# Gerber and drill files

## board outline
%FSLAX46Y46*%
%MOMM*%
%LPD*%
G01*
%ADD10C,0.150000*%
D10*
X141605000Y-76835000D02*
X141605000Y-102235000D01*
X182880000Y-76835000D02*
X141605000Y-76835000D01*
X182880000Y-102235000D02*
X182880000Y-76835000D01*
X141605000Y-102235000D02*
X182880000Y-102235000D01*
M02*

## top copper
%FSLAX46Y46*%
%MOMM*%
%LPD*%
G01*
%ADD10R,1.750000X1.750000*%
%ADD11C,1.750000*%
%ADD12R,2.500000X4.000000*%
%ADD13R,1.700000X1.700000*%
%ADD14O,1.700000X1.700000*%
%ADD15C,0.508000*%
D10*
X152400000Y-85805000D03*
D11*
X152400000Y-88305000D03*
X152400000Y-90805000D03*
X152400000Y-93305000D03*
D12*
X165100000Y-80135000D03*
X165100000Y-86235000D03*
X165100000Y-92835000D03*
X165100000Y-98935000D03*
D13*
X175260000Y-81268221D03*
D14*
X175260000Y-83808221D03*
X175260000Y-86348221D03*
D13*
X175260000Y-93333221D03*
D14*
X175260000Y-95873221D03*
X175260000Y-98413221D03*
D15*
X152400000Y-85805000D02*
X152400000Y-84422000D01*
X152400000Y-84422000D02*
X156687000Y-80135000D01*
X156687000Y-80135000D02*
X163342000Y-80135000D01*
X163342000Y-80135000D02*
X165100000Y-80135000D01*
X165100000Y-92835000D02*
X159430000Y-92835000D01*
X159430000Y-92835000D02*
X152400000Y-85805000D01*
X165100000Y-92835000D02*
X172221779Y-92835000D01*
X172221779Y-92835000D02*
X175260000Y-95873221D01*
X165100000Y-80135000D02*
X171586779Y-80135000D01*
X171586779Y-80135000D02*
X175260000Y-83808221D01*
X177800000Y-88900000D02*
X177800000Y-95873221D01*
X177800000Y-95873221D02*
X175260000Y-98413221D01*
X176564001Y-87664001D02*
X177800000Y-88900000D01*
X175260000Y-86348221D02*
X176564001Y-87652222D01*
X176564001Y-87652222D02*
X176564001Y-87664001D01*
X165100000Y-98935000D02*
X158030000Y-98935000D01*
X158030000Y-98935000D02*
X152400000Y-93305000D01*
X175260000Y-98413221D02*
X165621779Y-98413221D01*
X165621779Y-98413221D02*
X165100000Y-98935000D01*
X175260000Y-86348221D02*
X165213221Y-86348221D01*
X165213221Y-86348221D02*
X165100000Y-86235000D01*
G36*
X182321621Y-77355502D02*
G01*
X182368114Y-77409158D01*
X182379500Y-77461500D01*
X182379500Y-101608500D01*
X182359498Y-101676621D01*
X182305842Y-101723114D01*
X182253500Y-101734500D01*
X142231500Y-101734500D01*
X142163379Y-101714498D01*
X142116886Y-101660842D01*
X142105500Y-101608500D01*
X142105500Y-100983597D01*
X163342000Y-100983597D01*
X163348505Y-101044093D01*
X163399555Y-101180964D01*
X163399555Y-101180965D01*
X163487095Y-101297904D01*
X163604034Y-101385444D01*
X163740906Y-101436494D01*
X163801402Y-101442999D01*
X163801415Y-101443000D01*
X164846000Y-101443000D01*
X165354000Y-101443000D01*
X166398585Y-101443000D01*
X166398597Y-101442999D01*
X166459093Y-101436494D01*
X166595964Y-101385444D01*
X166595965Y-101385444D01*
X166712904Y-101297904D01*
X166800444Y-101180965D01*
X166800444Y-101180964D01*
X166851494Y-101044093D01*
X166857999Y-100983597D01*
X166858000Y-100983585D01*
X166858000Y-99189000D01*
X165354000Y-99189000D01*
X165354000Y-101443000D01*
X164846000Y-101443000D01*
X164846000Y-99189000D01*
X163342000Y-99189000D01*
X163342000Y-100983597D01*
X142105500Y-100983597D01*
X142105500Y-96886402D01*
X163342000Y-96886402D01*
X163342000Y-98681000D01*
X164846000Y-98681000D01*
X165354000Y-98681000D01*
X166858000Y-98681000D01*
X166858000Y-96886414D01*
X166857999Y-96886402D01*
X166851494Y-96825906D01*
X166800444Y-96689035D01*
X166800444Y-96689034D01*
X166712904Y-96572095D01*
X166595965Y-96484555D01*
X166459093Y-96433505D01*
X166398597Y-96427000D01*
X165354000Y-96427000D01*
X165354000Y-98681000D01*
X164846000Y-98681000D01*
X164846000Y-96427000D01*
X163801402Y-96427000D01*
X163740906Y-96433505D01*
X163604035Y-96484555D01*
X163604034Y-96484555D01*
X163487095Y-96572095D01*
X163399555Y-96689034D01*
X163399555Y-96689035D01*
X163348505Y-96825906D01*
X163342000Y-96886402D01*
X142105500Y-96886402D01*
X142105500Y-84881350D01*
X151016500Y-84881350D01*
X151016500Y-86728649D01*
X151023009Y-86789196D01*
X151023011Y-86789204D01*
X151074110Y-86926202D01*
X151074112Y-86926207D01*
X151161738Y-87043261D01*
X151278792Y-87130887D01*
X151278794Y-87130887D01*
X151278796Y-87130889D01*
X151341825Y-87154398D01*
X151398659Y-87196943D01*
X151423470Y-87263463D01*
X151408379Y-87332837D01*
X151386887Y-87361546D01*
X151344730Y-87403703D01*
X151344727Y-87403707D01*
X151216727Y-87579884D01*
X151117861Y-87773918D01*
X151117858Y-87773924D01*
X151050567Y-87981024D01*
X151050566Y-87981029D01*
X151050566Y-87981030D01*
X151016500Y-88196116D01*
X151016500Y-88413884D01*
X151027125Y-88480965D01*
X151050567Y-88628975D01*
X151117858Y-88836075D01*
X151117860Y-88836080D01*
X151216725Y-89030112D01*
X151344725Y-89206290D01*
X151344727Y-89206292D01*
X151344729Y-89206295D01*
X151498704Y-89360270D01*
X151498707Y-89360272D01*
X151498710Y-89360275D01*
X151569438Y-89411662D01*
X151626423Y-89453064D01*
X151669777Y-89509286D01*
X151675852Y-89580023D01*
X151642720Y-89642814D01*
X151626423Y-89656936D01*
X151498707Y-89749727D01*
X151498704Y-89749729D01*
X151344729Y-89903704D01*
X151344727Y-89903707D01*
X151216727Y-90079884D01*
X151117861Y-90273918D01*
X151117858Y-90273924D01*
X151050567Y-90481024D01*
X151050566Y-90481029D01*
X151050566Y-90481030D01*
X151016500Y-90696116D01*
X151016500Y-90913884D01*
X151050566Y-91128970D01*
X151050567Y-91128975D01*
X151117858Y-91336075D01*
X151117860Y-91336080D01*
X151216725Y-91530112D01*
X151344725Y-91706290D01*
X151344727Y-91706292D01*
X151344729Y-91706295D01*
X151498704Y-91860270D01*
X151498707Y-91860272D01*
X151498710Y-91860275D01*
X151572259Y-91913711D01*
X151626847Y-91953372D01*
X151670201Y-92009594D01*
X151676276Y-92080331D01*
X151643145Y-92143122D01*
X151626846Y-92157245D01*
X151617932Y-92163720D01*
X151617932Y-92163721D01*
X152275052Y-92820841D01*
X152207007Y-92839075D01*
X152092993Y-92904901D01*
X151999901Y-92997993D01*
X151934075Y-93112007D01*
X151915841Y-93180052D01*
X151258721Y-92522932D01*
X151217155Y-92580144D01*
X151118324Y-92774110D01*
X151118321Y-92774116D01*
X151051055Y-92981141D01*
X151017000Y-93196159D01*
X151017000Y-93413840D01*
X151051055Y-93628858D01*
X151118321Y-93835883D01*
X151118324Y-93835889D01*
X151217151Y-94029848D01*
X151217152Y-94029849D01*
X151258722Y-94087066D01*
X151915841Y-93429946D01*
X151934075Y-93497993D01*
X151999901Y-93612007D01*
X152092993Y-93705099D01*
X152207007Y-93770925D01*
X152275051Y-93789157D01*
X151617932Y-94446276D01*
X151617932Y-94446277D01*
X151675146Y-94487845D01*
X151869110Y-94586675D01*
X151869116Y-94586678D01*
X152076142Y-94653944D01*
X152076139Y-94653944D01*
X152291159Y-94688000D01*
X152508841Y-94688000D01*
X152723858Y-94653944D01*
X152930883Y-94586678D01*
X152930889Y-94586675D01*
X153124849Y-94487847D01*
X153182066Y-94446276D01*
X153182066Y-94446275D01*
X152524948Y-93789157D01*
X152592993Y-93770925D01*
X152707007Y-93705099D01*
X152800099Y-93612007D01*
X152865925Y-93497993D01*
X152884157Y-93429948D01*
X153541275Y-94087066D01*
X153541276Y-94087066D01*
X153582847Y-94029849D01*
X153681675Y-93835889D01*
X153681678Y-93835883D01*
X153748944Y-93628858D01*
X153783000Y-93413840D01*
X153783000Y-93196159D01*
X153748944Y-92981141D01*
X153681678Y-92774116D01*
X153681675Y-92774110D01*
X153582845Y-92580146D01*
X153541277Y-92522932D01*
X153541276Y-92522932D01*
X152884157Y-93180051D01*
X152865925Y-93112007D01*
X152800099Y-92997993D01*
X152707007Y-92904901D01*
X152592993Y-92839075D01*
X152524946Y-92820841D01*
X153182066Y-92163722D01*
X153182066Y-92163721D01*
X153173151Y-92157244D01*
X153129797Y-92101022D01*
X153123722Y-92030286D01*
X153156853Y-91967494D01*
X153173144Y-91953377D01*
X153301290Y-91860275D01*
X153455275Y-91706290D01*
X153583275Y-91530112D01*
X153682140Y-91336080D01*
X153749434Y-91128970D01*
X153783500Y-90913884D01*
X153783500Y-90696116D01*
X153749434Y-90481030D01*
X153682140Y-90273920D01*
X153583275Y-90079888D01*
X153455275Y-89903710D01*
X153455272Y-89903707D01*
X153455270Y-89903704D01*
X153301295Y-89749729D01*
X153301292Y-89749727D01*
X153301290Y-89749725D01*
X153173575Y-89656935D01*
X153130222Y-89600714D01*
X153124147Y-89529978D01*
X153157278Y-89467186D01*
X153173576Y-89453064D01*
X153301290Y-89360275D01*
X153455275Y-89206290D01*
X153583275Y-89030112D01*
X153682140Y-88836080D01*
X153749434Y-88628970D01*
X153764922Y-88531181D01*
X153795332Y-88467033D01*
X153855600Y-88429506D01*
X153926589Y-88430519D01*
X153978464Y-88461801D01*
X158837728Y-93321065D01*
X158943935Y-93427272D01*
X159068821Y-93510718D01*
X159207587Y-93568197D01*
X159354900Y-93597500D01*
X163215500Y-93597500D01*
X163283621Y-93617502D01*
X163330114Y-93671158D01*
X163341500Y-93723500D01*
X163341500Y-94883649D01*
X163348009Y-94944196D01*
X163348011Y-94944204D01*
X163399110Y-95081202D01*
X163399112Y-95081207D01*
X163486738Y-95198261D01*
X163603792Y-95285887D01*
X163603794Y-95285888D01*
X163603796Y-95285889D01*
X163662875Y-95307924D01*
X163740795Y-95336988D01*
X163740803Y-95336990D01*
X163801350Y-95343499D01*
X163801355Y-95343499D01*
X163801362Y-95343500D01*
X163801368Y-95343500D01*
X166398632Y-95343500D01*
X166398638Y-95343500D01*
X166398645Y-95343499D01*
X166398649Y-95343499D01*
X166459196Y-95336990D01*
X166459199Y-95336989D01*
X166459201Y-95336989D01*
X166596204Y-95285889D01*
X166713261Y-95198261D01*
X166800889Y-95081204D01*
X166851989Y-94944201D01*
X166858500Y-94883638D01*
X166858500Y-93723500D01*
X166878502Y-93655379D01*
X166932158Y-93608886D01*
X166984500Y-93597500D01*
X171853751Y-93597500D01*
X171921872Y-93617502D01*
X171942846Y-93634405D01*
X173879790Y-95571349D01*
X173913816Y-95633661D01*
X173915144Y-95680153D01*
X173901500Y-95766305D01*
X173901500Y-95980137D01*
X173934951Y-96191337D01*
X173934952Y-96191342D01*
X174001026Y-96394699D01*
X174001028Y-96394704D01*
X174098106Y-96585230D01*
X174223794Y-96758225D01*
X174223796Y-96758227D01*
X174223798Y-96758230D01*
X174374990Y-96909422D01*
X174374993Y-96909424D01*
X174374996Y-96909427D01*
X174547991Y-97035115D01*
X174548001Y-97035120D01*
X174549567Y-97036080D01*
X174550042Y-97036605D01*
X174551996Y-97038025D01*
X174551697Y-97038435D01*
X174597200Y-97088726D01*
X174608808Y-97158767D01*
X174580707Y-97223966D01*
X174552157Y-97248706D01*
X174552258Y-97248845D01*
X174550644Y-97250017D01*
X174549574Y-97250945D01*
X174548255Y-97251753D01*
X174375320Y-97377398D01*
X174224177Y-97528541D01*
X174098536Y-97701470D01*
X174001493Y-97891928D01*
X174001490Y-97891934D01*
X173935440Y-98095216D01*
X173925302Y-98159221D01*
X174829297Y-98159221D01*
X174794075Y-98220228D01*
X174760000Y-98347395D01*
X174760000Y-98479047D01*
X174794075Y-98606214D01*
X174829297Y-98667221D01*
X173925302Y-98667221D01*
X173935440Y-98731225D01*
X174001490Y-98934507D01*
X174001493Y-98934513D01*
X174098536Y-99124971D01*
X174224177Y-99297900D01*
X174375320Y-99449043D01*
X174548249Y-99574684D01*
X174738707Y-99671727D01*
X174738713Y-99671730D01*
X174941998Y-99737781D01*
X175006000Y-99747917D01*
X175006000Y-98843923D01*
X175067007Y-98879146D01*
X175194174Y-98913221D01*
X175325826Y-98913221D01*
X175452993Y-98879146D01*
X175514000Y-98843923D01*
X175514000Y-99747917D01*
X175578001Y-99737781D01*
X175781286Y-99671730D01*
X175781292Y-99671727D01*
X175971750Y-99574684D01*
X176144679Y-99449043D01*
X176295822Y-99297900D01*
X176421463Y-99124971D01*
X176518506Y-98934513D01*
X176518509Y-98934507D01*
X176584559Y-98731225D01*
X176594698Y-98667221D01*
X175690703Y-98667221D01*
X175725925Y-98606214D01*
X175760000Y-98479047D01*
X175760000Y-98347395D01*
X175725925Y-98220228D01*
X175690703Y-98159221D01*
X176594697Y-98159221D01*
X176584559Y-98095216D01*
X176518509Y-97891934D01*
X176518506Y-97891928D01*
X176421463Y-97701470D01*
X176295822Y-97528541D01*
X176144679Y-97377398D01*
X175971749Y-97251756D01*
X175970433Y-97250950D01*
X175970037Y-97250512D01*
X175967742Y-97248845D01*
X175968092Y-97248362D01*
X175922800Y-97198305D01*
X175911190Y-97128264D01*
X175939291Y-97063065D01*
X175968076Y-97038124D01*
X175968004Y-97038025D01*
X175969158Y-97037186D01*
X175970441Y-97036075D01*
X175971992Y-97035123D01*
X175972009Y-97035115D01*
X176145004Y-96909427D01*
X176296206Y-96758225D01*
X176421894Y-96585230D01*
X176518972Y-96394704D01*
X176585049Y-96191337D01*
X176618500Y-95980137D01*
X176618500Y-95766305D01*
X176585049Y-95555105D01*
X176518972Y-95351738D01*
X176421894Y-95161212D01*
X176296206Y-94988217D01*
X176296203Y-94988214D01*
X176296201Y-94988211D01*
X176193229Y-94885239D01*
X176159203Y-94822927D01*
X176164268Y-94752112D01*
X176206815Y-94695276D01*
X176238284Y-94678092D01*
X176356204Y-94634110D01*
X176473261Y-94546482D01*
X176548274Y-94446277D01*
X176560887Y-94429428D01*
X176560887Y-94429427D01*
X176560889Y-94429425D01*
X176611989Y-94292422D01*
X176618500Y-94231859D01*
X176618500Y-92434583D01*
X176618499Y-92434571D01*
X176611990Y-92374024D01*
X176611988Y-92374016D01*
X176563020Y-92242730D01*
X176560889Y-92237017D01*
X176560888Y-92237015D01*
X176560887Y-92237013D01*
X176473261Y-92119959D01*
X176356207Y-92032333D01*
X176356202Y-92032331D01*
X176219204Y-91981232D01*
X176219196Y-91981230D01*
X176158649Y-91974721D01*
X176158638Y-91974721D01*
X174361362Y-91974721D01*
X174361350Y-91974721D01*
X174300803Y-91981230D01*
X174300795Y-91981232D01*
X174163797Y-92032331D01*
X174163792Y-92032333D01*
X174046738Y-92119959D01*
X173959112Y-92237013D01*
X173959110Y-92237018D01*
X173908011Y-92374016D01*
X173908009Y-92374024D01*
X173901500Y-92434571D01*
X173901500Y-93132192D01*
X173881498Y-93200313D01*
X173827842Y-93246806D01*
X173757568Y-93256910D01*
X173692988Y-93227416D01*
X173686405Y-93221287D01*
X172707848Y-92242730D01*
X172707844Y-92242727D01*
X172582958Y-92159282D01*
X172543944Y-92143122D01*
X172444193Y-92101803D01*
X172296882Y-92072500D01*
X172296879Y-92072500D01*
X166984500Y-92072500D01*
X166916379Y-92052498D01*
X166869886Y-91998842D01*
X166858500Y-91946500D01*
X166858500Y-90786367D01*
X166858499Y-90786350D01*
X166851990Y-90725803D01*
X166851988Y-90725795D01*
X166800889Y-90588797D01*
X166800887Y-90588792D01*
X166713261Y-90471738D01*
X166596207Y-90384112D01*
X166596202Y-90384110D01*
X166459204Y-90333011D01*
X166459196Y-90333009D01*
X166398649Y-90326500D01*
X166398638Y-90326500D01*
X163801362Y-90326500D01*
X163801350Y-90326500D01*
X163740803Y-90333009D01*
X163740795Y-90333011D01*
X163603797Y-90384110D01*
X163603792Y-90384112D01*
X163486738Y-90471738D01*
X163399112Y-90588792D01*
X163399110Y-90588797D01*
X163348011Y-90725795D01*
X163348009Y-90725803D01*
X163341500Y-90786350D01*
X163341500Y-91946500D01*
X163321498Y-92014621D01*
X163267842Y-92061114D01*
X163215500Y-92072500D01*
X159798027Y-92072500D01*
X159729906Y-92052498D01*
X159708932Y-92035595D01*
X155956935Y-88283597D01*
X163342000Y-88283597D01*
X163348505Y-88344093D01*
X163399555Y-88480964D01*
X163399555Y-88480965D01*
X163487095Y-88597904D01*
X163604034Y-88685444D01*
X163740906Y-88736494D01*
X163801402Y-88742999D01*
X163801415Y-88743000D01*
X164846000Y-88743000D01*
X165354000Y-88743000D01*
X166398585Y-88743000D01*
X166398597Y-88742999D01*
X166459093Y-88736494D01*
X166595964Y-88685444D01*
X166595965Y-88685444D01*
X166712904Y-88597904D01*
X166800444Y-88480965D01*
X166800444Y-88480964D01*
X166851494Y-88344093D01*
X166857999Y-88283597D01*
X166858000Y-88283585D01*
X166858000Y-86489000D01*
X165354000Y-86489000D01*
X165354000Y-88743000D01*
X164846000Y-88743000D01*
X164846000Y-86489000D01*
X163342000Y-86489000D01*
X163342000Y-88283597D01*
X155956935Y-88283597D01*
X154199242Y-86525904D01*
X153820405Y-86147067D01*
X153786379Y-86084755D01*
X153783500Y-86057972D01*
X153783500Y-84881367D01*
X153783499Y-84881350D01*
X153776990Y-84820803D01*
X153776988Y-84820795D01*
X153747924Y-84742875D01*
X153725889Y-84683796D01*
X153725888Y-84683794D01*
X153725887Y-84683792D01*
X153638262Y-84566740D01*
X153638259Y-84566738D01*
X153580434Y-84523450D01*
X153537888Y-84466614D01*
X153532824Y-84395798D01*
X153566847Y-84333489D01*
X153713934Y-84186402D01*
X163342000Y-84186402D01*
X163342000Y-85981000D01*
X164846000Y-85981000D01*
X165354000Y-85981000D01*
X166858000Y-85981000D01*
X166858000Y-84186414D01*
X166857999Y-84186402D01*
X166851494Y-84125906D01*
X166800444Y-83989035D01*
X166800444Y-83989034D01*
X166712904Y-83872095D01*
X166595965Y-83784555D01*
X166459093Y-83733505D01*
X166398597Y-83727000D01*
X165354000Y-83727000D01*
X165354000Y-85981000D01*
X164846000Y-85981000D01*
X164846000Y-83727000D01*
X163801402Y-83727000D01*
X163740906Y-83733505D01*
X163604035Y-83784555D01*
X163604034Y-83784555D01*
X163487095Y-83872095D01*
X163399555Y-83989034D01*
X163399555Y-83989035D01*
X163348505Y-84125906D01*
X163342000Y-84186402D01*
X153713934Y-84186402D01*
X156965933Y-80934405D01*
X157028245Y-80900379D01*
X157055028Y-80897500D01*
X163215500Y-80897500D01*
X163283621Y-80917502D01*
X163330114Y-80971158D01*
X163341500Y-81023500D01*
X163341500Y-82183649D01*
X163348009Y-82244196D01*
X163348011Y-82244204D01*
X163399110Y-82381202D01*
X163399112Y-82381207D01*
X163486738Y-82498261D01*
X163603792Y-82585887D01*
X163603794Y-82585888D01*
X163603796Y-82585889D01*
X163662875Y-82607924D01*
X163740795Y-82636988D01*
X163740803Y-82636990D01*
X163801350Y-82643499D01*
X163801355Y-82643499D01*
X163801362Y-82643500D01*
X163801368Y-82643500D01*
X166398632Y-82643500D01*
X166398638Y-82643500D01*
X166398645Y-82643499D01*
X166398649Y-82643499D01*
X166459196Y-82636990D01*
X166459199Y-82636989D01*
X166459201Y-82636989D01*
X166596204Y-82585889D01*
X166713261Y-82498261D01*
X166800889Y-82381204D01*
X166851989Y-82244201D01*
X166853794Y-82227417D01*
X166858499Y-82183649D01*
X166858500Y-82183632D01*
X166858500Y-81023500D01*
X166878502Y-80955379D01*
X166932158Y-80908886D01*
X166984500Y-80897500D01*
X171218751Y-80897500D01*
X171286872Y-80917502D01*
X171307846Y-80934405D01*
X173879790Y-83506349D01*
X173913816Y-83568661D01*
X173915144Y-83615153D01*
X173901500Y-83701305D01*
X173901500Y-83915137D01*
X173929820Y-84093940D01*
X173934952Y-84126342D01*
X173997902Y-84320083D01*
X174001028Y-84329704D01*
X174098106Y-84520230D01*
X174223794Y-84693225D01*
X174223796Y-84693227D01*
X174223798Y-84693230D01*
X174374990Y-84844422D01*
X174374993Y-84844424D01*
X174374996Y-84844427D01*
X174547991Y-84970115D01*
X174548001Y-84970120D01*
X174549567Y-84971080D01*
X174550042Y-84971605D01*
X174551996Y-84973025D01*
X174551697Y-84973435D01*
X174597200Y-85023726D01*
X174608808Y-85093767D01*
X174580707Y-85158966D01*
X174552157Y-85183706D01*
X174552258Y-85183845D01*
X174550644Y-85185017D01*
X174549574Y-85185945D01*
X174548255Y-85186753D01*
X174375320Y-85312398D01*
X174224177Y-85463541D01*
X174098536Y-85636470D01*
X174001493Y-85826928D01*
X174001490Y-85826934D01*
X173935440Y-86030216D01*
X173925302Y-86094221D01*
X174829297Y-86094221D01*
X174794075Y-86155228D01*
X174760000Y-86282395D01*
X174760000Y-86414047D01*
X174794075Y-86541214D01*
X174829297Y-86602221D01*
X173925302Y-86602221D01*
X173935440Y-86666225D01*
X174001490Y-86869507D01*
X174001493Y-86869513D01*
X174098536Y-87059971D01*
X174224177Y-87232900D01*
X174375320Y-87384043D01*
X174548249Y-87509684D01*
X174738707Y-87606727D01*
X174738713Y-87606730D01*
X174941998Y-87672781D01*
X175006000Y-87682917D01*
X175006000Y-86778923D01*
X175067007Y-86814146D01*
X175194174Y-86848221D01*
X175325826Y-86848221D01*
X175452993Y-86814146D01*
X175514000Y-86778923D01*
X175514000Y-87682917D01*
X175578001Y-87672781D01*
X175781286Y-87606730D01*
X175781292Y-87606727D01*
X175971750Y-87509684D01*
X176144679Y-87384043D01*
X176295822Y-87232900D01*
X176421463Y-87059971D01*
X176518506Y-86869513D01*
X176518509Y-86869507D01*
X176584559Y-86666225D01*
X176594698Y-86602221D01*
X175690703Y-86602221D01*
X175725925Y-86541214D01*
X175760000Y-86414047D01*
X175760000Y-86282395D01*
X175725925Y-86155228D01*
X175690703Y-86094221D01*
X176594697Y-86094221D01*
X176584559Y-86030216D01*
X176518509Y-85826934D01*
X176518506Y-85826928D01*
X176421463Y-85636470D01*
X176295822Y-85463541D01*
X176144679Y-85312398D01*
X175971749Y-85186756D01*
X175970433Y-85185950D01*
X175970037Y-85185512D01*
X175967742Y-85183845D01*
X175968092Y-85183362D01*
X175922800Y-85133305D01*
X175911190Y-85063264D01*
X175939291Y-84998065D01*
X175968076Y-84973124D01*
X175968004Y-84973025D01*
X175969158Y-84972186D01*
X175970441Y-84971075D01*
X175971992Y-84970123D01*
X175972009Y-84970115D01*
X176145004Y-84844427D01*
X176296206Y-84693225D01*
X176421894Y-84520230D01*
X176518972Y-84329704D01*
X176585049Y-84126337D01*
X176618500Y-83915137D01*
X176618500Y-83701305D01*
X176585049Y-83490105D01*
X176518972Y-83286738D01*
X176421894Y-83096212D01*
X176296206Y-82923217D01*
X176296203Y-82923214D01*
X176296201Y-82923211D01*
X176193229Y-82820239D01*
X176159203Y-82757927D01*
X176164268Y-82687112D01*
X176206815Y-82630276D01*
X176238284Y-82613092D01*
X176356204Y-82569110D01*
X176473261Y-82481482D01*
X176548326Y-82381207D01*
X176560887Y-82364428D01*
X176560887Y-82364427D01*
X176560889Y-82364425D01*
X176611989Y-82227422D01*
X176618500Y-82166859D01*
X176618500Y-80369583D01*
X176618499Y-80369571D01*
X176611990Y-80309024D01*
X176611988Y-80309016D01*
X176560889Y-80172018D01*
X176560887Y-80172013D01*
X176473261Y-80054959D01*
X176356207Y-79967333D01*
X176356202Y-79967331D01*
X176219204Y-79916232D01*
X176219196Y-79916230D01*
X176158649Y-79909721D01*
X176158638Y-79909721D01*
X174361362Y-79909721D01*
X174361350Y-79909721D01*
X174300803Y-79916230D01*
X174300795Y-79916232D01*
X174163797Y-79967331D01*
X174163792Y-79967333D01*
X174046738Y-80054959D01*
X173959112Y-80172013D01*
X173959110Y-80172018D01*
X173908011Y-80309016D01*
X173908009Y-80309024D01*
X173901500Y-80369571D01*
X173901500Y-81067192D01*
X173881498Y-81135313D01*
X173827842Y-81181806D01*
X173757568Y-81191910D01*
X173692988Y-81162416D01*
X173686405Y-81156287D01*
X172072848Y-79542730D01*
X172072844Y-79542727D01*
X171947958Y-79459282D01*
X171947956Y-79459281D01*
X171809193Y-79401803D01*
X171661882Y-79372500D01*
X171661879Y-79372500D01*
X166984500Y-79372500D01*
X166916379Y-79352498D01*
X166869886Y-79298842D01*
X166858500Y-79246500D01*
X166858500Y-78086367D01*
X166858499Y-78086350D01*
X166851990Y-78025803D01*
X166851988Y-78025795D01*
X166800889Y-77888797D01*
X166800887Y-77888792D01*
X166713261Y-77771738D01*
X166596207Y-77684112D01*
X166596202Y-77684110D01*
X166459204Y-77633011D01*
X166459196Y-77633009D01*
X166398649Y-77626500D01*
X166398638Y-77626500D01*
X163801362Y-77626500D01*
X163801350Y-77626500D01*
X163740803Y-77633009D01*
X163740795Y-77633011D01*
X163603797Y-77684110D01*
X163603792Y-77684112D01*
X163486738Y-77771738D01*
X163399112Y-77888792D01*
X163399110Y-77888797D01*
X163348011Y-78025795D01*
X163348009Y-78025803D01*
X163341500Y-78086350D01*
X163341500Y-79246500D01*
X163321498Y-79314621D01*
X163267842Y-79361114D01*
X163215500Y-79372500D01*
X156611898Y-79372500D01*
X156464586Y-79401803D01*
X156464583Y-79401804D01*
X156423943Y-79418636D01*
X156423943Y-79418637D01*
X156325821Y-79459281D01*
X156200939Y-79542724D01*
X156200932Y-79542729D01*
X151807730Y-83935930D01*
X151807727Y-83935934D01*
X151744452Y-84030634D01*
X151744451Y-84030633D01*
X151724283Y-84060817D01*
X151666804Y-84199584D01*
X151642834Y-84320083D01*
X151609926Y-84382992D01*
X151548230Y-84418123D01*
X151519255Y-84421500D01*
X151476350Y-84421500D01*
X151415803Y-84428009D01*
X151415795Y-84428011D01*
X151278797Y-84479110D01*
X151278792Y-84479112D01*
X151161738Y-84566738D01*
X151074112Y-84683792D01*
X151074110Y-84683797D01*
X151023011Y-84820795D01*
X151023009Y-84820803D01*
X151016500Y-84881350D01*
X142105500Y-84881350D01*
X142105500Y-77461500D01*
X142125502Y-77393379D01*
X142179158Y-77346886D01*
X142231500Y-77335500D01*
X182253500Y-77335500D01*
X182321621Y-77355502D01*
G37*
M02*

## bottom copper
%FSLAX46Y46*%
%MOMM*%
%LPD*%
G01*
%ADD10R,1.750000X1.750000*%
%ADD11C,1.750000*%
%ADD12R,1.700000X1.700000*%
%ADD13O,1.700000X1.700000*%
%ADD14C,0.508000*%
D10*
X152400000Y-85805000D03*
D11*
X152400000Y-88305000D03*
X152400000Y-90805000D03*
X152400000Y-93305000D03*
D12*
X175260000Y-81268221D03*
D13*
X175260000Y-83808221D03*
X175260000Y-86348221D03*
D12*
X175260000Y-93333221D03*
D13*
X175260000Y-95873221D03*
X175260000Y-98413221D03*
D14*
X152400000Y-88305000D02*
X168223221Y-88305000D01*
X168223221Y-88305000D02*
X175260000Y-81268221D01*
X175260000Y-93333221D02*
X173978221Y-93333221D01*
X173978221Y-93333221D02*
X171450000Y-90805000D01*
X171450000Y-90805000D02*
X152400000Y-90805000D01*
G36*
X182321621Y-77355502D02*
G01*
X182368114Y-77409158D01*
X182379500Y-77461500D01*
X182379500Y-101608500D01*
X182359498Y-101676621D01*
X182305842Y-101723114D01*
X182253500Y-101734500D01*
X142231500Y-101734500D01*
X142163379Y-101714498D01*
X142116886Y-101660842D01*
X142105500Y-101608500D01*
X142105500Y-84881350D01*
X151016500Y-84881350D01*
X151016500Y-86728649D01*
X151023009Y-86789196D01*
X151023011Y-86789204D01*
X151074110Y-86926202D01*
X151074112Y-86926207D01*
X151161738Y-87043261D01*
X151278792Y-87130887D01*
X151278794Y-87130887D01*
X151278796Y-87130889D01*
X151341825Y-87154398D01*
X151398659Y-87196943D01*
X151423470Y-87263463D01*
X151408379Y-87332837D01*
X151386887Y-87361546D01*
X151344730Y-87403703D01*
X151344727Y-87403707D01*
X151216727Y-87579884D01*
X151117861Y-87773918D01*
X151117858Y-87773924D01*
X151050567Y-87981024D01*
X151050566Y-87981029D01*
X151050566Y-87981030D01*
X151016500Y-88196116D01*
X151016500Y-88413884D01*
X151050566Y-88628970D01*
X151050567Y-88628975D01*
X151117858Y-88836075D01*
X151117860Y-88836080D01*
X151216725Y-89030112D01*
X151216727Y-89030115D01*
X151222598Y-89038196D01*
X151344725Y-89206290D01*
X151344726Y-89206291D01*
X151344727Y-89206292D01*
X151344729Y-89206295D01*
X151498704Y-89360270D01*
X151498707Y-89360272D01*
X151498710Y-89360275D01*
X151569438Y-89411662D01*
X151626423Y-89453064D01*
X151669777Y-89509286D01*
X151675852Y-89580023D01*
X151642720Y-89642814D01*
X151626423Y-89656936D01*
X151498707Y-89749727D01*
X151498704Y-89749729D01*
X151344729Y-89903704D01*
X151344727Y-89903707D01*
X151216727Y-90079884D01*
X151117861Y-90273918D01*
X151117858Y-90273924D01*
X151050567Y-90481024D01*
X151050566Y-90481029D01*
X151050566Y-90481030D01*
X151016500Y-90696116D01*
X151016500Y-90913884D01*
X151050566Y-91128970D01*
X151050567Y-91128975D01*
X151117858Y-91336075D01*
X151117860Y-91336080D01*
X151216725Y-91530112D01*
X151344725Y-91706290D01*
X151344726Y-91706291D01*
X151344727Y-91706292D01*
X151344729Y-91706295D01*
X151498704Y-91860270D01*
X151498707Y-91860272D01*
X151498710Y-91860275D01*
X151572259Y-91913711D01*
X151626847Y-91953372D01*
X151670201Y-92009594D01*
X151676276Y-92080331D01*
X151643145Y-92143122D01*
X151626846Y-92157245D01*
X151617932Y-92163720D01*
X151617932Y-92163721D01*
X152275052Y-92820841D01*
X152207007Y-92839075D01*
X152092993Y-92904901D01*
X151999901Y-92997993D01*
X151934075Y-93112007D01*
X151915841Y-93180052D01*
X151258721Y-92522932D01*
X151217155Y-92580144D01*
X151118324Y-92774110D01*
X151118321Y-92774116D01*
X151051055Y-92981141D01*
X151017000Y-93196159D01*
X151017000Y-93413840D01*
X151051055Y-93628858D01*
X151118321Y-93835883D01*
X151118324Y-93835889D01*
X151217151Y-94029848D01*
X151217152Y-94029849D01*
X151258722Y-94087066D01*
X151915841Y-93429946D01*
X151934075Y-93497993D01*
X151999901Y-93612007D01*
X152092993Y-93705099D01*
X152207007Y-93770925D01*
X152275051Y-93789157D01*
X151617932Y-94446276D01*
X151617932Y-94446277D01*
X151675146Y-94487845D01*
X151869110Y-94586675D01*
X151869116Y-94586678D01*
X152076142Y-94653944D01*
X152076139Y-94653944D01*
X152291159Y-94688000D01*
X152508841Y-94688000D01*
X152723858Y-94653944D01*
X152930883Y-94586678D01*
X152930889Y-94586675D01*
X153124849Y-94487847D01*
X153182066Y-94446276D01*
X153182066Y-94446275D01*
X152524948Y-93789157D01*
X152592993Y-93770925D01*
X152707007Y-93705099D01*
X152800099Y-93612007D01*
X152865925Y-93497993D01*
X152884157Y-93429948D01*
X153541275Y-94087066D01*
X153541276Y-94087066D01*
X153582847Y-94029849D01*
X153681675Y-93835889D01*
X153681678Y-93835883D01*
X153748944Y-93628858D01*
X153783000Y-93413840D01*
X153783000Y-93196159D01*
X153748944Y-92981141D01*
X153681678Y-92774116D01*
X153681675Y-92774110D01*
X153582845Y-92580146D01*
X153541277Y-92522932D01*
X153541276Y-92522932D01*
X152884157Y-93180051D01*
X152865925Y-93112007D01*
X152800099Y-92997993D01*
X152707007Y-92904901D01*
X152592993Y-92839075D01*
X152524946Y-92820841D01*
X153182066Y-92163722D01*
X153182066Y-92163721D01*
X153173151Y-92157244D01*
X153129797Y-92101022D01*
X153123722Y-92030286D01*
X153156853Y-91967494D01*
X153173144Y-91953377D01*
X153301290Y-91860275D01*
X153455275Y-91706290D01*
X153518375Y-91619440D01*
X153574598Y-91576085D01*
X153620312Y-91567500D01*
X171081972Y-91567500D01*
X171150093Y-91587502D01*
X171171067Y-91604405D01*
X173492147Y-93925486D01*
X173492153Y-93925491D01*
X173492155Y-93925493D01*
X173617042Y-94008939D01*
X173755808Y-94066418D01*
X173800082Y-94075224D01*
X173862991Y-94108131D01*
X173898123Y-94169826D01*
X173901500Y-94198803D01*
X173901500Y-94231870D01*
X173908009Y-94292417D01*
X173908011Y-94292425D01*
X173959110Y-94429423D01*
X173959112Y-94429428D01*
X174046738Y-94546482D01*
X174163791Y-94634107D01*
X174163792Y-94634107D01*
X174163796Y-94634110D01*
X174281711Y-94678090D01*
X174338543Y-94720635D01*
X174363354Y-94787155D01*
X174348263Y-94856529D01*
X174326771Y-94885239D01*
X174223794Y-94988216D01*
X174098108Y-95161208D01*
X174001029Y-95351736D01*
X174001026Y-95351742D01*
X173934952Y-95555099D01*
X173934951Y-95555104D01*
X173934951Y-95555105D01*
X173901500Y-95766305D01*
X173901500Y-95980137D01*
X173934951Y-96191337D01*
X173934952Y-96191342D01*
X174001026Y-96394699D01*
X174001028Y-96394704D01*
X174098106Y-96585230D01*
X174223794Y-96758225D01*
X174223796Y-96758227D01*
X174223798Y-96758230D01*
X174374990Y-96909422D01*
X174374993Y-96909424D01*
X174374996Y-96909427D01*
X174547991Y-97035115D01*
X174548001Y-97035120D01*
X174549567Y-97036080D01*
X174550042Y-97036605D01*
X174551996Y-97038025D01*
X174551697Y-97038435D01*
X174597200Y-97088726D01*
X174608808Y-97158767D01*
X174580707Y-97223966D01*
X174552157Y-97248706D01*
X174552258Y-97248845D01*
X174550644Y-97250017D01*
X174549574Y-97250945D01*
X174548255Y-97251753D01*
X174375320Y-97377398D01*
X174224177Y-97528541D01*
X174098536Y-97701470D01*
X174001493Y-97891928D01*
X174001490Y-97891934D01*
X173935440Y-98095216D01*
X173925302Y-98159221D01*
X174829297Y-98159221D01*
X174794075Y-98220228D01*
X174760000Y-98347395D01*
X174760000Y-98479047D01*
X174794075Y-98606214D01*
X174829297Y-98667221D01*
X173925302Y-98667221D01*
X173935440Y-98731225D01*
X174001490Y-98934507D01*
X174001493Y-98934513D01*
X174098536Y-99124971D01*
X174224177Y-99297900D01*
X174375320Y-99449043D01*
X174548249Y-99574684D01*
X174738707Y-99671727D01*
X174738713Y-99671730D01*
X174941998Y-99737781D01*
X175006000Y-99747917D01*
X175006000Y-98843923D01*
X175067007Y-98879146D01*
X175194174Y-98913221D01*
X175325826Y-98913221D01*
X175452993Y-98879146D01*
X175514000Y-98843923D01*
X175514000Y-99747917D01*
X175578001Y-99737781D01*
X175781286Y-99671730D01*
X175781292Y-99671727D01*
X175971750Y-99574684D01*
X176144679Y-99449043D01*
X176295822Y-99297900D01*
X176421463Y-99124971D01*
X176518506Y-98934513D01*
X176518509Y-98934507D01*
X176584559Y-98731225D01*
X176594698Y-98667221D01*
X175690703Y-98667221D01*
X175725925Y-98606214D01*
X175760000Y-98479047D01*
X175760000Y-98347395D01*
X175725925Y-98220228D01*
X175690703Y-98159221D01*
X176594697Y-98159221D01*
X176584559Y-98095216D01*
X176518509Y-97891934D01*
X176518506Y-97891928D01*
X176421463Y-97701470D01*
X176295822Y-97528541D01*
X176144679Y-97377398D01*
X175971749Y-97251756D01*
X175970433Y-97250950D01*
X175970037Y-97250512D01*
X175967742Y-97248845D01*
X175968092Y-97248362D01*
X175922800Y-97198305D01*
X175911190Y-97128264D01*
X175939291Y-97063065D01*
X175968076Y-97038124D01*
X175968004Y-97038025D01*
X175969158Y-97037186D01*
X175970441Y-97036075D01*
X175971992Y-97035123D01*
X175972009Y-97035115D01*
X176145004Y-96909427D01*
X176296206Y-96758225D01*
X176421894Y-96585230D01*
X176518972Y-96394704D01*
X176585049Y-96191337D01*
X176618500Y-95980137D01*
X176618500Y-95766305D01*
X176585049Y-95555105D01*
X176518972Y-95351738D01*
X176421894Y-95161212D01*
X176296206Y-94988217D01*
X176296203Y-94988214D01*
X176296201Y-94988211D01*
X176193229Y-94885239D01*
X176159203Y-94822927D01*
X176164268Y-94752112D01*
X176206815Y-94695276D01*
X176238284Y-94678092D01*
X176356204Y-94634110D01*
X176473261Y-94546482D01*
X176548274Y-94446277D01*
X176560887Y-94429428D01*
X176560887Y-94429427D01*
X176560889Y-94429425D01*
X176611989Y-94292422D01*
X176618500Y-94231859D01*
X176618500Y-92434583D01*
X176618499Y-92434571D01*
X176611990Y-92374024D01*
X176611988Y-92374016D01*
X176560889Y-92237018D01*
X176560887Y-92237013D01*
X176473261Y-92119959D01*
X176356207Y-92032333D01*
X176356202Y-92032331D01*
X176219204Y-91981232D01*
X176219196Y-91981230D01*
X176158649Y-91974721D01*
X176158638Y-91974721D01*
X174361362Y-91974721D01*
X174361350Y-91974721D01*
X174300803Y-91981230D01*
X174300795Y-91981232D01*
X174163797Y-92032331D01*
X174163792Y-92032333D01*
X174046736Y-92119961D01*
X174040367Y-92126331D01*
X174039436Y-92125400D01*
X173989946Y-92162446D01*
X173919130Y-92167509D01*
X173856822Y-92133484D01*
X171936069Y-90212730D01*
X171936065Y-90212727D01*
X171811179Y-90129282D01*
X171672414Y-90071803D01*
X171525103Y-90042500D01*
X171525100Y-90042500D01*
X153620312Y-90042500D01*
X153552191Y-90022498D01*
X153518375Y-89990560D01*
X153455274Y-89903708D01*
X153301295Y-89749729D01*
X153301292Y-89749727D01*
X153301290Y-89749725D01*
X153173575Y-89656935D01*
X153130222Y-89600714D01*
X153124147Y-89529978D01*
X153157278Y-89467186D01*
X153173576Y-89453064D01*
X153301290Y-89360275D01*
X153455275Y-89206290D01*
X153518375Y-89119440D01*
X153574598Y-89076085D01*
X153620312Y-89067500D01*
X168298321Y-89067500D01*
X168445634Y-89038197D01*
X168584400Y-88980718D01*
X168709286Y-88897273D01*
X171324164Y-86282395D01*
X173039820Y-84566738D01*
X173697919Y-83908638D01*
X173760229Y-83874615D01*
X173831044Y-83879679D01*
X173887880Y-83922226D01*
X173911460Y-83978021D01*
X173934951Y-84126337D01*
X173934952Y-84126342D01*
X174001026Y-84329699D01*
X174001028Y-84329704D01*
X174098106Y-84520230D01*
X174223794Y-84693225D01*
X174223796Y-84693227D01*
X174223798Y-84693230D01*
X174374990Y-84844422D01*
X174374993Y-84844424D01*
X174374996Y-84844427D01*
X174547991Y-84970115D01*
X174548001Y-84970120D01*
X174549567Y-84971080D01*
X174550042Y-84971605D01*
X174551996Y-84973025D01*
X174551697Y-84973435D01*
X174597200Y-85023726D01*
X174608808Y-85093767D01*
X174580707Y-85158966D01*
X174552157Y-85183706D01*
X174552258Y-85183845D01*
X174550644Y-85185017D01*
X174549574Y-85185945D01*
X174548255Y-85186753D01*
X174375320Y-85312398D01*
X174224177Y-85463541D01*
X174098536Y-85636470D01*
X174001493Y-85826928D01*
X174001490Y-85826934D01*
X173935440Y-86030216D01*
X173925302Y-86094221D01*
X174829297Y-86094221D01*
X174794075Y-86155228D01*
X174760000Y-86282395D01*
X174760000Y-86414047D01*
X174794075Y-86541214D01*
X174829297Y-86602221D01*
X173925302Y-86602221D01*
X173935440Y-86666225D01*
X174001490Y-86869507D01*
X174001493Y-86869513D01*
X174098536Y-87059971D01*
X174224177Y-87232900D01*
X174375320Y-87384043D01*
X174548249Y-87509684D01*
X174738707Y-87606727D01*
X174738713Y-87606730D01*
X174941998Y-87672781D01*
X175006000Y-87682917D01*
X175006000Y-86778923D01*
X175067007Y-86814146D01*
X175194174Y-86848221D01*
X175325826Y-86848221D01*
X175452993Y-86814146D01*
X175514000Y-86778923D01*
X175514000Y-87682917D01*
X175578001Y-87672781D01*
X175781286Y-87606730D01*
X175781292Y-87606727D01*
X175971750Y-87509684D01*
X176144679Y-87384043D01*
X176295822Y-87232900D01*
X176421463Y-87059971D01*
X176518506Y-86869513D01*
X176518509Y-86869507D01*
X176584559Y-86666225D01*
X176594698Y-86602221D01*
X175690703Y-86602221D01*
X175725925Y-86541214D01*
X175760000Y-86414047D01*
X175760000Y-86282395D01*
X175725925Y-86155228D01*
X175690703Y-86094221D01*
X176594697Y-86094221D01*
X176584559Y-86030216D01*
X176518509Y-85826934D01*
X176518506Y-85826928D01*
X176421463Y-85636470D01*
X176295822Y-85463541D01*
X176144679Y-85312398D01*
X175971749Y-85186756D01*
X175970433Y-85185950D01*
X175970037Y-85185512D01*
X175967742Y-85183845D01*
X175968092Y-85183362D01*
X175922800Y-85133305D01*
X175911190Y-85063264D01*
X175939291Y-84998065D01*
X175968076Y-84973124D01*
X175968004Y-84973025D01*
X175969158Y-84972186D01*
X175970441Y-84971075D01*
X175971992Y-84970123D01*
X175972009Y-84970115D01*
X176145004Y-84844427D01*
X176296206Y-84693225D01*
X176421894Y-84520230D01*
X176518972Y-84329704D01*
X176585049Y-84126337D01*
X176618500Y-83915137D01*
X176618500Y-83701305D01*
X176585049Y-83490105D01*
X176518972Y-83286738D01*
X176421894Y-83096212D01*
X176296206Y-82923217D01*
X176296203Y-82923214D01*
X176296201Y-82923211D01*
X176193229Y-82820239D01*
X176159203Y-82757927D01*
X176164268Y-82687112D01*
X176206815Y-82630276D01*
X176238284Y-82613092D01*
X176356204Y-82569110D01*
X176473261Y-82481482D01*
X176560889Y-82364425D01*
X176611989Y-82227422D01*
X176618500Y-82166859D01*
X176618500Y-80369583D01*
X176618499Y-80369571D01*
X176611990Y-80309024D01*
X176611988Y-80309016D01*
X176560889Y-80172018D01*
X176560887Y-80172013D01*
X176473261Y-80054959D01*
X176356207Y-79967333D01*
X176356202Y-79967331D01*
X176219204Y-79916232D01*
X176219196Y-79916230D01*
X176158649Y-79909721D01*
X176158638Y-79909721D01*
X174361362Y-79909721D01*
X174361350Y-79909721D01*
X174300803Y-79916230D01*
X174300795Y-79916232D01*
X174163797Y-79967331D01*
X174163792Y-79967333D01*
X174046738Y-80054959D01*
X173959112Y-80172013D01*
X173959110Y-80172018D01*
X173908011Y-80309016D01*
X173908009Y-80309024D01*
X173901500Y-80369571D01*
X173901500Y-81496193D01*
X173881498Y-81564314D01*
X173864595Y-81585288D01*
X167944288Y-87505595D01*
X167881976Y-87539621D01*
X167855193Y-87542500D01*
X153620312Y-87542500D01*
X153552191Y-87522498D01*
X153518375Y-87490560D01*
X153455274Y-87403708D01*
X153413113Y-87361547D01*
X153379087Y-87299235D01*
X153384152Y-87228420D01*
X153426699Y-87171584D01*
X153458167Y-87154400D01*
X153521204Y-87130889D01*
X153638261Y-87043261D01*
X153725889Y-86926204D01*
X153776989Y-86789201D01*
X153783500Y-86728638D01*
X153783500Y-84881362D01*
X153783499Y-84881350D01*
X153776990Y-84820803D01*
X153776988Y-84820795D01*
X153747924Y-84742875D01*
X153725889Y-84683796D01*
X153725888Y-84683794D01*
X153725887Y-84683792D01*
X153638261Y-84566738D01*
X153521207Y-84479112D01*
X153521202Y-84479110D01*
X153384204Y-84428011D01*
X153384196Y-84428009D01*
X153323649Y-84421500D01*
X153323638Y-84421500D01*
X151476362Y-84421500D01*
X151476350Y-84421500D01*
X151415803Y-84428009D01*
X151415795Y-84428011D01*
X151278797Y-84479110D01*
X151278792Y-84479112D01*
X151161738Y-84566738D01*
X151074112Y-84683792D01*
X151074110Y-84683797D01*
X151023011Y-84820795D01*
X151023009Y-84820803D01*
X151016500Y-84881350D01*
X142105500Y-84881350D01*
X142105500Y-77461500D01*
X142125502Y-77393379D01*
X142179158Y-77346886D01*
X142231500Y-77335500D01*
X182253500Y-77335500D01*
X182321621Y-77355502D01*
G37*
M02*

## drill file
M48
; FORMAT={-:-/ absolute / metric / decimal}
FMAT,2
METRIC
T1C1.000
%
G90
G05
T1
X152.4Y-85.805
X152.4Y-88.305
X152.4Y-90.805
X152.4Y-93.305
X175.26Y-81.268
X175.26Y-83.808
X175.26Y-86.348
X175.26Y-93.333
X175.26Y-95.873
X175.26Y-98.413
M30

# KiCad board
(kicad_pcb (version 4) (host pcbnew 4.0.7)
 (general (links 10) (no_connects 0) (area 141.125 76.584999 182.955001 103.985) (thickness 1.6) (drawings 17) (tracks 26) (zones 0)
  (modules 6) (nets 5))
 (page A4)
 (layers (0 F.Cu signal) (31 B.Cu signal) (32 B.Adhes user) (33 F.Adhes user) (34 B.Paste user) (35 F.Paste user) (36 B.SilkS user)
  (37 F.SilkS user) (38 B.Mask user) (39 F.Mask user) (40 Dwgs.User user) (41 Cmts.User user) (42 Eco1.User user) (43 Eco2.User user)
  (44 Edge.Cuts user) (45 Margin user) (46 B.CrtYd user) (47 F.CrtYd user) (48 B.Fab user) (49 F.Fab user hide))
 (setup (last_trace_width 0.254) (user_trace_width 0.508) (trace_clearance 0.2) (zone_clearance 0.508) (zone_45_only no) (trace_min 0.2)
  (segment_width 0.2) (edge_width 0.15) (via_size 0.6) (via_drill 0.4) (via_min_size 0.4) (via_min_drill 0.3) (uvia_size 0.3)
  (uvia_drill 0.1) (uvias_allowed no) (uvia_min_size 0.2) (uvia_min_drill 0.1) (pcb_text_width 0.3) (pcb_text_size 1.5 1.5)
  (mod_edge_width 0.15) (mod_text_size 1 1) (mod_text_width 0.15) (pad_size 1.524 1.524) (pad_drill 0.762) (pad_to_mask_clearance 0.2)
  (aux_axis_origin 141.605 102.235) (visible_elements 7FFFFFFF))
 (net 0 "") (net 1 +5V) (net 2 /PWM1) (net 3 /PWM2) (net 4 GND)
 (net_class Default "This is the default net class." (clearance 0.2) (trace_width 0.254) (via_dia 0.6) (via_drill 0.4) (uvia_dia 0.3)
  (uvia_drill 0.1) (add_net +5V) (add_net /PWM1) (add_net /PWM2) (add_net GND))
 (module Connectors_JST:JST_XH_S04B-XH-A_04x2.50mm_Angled (layer F.Cu) (at 152.4 85.805 270)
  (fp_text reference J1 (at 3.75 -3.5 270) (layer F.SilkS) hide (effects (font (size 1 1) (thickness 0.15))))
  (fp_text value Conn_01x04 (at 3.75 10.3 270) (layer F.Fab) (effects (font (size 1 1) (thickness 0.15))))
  (pad 1 thru_hole rect (at 0 0 270) (size 1.75 1.75) (drill 1) (layers *.Cu *.Mask F.SilkS) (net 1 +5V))
  (pad 2 thru_hole circle (at 2.5 0 270) (size 1.75 1.75) (drill 1) (layers *.Cu *.Mask F.SilkS) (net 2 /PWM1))
  (pad 3 thru_hole circle (at 5 0 270) (size 1.75 1.75) (drill 1) (layers *.Cu *.Mask F.SilkS) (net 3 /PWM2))
  (pad 4 thru_hole circle (at 7.5 0 270) (size 1.75 1.75) (drill 1) (layers *.Cu *.Mask F.SilkS) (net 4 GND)))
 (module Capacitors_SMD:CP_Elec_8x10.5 (layer F.Cu) (at 165.1 83.185 270)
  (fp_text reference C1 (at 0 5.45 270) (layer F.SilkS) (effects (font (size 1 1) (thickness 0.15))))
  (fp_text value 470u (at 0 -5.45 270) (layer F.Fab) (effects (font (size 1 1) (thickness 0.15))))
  (pad 1 smd rect (at -3.05 0 90) (size 4 2.5) (layers F.Cu F.Paste F.Mask) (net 1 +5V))
  (pad 2 smd rect (at 3.05 0 90) (size 4 2.5) (layers F.Cu F.Paste F.Mask) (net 4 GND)))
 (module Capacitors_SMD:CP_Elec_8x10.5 (layer F.Cu) (at 165.1 95.885 270)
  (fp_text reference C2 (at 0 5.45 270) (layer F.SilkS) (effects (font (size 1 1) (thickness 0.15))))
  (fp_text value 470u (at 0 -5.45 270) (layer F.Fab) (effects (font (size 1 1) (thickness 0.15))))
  (pad 1 smd rect (at -3.05 0 90) (size 4 2.5) (layers F.Cu F.Paste F.Mask) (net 1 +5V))
  (pad 2 smd rect (at 3.05 0 90) (size 4 2.5) (layers F.Cu F.Paste F.Mask) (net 4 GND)))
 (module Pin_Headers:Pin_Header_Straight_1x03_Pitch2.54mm (layer F.Cu) (at 175.26 81.268221)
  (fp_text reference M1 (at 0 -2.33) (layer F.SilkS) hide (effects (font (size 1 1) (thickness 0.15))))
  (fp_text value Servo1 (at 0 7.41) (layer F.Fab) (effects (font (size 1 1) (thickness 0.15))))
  (pad 1 thru_hole rect (at 0 0) (size 1.7 1.7) (drill 1) (layers *.Cu *.Mask) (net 2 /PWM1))
  (pad 2 thru_hole oval (at 0 2.54) (size 1.7 1.7) (drill 1) (layers *.Cu *.Mask) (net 1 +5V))
  (pad 3 thru_hole oval (at 0 5.08) (size 1.7 1.7) (drill 1) (layers *.Cu *.Mask) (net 4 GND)))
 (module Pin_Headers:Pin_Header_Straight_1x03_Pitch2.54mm (layer F.Cu) (at 175.26 93.333221)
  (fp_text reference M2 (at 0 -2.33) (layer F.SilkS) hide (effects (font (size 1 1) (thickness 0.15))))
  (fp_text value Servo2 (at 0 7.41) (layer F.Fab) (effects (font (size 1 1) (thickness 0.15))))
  (pad 1 thru_hole rect (at 0 0) (size 1.7 1.7) (drill 1) (layers *.Cu *.Mask) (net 3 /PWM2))
  (pad 2 thru_hole oval (at 0 2.54) (size 1.7 1.7) (drill 1) (layers *.Cu *.Mask) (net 1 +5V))
  (pad 3 thru_hole oval (at 0 5.08) (size 1.7 1.7) (drill 1) (layers *.Cu *.Mask) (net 4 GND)))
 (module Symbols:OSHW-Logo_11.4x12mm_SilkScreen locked (layer B.Cu) (at 166.37 89.535 270)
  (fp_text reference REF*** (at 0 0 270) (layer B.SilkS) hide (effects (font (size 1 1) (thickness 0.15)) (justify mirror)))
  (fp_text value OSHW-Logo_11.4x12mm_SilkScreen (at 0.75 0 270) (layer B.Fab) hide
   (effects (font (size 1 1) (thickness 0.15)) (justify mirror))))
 (gr_line (start 141.605 76.835) (end 141.605 102.235) (layer Edge.Cuts) (width 0.15))
 (gr_line (start 182.88 76.835) (end 141.605 76.835) (layer Edge.Cuts) (width 0.15))
 (gr_line (start 182.88 102.235) (end 182.88 76.835) (layer Edge.Cuts) (width 0.15))
 (gr_line (start 141.605 102.235) (end 182.88 102.235) (layer Edge.Cuts) (width 0.15))
 (segment (start 152.4 85.805) (end 152.4 84.422) (width 0.508) (layer F.Cu) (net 1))
 (segment (start 152.4 84.422) (end 156.687 80.135) (width 0.508) (layer F.Cu) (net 1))
 (segment (start 156.687 80.135) (end 163.342 80.135) (width 0.508) (layer F.Cu) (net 1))
 (segment (start 163.342 80.135) (end 165.1 80.135) (width 0.508) (layer F.Cu) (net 1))
 (segment (start 165.1 92.835) (end 159.43 92.835) (width 0.508) (layer F.Cu) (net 1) (status 10))
 (segment (start 159.43 92.835) (end 152.4 85.805) (width 0.508) (layer F.Cu) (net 1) (status 20))
 (segment (start 165.1 92.835) (end 172.221779 92.835) (width 0.508) (layer F.Cu) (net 1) (status 10))
 (segment (start 172.221779 92.835) (end 175.26 95.873221) (width 0.508) (layer F.Cu) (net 1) (status 20))
 (segment (start 165.1 80.135) (end 171.586779 80.135) (width 0.508) (layer F.Cu) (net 1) (status 10))
 (segment (start 171.586779 80.135) (end 175.26 83.808221) (width 0.508) (layer F.Cu) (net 1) (status 20))
 (segment (start 177.8 88.9) (end 177.8 95.873221) (width 0.508) (layer F.Cu) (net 4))
 (segment (start 177.8 95.873221) (end 175.26 98.413221) (width 0.508) (layer F.Cu) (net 4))
 (segment (start 176.564001 87.664001) (end 177.8 88.9) (width 0.508) (layer F.Cu) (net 4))
 (segment (start 175.26 86.348221) (end 176.564001 87.652222) (width 0.508) (layer F.Cu) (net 4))
 (segment (start 176.564001 87.652222) (end 176.564001 87.664001) (width 0.508) (layer F.Cu) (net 4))
 (segment (start 165.1 98.935) (end 158.03 98.935) (width 0.508) (layer F.Cu) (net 4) (status 10))
 (segment (start 158.03 98.935) (end 152.4 93.305) (width 0.508) (layer F.Cu) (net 4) (status 20))
 (segment (start 175.26 98.413221) (end 165.621779 98.413221) (width 0.508) (layer F.Cu) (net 4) (status 30))
 (segment (start 165.621779 98.413221) (end 165.1 98.935) (width 0.508) (layer F.Cu) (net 4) (status 30))
 (segment (start 175.26 86.348221) (end 165.213221 86.348221) (width 0.508) (layer F.Cu) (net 4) (status 30))
 (segment (start 165.213221 86.348221) (end 165.1 86.235) (width 0.508) (layer F.Cu) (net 4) (status 30))
 (segment (start 152.4 88.305) (end 168.223221 88.305) (width 0.508) (layer B.Cu) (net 2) (status 10))
 (segment (start 168.223221 88.305) (end 175.26 81.268221) (width 0.508) (layer B.Cu) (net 2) (status 20))
 (segment (start 175.26 93.333221) (end 173.978221 93.333221) (width 0.508) (layer B.Cu) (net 3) (status 10))
 (segment (start 173.978221 93.333221) (end 171.45 90.805) (width 0.508) (layer B.Cu) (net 3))
 (segment (start 171.45 90.805) (end 152.4 90.805) (width 0.508) (layer B.Cu) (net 3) (status 20))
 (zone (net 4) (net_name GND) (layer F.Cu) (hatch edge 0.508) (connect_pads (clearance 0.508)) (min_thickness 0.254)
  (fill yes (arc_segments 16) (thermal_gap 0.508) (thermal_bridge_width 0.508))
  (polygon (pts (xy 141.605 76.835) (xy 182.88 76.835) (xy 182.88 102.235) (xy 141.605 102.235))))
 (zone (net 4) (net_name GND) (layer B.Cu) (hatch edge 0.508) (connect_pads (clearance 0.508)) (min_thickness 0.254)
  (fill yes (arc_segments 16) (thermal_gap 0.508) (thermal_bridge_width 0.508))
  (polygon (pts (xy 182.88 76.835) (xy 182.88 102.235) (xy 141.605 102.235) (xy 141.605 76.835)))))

